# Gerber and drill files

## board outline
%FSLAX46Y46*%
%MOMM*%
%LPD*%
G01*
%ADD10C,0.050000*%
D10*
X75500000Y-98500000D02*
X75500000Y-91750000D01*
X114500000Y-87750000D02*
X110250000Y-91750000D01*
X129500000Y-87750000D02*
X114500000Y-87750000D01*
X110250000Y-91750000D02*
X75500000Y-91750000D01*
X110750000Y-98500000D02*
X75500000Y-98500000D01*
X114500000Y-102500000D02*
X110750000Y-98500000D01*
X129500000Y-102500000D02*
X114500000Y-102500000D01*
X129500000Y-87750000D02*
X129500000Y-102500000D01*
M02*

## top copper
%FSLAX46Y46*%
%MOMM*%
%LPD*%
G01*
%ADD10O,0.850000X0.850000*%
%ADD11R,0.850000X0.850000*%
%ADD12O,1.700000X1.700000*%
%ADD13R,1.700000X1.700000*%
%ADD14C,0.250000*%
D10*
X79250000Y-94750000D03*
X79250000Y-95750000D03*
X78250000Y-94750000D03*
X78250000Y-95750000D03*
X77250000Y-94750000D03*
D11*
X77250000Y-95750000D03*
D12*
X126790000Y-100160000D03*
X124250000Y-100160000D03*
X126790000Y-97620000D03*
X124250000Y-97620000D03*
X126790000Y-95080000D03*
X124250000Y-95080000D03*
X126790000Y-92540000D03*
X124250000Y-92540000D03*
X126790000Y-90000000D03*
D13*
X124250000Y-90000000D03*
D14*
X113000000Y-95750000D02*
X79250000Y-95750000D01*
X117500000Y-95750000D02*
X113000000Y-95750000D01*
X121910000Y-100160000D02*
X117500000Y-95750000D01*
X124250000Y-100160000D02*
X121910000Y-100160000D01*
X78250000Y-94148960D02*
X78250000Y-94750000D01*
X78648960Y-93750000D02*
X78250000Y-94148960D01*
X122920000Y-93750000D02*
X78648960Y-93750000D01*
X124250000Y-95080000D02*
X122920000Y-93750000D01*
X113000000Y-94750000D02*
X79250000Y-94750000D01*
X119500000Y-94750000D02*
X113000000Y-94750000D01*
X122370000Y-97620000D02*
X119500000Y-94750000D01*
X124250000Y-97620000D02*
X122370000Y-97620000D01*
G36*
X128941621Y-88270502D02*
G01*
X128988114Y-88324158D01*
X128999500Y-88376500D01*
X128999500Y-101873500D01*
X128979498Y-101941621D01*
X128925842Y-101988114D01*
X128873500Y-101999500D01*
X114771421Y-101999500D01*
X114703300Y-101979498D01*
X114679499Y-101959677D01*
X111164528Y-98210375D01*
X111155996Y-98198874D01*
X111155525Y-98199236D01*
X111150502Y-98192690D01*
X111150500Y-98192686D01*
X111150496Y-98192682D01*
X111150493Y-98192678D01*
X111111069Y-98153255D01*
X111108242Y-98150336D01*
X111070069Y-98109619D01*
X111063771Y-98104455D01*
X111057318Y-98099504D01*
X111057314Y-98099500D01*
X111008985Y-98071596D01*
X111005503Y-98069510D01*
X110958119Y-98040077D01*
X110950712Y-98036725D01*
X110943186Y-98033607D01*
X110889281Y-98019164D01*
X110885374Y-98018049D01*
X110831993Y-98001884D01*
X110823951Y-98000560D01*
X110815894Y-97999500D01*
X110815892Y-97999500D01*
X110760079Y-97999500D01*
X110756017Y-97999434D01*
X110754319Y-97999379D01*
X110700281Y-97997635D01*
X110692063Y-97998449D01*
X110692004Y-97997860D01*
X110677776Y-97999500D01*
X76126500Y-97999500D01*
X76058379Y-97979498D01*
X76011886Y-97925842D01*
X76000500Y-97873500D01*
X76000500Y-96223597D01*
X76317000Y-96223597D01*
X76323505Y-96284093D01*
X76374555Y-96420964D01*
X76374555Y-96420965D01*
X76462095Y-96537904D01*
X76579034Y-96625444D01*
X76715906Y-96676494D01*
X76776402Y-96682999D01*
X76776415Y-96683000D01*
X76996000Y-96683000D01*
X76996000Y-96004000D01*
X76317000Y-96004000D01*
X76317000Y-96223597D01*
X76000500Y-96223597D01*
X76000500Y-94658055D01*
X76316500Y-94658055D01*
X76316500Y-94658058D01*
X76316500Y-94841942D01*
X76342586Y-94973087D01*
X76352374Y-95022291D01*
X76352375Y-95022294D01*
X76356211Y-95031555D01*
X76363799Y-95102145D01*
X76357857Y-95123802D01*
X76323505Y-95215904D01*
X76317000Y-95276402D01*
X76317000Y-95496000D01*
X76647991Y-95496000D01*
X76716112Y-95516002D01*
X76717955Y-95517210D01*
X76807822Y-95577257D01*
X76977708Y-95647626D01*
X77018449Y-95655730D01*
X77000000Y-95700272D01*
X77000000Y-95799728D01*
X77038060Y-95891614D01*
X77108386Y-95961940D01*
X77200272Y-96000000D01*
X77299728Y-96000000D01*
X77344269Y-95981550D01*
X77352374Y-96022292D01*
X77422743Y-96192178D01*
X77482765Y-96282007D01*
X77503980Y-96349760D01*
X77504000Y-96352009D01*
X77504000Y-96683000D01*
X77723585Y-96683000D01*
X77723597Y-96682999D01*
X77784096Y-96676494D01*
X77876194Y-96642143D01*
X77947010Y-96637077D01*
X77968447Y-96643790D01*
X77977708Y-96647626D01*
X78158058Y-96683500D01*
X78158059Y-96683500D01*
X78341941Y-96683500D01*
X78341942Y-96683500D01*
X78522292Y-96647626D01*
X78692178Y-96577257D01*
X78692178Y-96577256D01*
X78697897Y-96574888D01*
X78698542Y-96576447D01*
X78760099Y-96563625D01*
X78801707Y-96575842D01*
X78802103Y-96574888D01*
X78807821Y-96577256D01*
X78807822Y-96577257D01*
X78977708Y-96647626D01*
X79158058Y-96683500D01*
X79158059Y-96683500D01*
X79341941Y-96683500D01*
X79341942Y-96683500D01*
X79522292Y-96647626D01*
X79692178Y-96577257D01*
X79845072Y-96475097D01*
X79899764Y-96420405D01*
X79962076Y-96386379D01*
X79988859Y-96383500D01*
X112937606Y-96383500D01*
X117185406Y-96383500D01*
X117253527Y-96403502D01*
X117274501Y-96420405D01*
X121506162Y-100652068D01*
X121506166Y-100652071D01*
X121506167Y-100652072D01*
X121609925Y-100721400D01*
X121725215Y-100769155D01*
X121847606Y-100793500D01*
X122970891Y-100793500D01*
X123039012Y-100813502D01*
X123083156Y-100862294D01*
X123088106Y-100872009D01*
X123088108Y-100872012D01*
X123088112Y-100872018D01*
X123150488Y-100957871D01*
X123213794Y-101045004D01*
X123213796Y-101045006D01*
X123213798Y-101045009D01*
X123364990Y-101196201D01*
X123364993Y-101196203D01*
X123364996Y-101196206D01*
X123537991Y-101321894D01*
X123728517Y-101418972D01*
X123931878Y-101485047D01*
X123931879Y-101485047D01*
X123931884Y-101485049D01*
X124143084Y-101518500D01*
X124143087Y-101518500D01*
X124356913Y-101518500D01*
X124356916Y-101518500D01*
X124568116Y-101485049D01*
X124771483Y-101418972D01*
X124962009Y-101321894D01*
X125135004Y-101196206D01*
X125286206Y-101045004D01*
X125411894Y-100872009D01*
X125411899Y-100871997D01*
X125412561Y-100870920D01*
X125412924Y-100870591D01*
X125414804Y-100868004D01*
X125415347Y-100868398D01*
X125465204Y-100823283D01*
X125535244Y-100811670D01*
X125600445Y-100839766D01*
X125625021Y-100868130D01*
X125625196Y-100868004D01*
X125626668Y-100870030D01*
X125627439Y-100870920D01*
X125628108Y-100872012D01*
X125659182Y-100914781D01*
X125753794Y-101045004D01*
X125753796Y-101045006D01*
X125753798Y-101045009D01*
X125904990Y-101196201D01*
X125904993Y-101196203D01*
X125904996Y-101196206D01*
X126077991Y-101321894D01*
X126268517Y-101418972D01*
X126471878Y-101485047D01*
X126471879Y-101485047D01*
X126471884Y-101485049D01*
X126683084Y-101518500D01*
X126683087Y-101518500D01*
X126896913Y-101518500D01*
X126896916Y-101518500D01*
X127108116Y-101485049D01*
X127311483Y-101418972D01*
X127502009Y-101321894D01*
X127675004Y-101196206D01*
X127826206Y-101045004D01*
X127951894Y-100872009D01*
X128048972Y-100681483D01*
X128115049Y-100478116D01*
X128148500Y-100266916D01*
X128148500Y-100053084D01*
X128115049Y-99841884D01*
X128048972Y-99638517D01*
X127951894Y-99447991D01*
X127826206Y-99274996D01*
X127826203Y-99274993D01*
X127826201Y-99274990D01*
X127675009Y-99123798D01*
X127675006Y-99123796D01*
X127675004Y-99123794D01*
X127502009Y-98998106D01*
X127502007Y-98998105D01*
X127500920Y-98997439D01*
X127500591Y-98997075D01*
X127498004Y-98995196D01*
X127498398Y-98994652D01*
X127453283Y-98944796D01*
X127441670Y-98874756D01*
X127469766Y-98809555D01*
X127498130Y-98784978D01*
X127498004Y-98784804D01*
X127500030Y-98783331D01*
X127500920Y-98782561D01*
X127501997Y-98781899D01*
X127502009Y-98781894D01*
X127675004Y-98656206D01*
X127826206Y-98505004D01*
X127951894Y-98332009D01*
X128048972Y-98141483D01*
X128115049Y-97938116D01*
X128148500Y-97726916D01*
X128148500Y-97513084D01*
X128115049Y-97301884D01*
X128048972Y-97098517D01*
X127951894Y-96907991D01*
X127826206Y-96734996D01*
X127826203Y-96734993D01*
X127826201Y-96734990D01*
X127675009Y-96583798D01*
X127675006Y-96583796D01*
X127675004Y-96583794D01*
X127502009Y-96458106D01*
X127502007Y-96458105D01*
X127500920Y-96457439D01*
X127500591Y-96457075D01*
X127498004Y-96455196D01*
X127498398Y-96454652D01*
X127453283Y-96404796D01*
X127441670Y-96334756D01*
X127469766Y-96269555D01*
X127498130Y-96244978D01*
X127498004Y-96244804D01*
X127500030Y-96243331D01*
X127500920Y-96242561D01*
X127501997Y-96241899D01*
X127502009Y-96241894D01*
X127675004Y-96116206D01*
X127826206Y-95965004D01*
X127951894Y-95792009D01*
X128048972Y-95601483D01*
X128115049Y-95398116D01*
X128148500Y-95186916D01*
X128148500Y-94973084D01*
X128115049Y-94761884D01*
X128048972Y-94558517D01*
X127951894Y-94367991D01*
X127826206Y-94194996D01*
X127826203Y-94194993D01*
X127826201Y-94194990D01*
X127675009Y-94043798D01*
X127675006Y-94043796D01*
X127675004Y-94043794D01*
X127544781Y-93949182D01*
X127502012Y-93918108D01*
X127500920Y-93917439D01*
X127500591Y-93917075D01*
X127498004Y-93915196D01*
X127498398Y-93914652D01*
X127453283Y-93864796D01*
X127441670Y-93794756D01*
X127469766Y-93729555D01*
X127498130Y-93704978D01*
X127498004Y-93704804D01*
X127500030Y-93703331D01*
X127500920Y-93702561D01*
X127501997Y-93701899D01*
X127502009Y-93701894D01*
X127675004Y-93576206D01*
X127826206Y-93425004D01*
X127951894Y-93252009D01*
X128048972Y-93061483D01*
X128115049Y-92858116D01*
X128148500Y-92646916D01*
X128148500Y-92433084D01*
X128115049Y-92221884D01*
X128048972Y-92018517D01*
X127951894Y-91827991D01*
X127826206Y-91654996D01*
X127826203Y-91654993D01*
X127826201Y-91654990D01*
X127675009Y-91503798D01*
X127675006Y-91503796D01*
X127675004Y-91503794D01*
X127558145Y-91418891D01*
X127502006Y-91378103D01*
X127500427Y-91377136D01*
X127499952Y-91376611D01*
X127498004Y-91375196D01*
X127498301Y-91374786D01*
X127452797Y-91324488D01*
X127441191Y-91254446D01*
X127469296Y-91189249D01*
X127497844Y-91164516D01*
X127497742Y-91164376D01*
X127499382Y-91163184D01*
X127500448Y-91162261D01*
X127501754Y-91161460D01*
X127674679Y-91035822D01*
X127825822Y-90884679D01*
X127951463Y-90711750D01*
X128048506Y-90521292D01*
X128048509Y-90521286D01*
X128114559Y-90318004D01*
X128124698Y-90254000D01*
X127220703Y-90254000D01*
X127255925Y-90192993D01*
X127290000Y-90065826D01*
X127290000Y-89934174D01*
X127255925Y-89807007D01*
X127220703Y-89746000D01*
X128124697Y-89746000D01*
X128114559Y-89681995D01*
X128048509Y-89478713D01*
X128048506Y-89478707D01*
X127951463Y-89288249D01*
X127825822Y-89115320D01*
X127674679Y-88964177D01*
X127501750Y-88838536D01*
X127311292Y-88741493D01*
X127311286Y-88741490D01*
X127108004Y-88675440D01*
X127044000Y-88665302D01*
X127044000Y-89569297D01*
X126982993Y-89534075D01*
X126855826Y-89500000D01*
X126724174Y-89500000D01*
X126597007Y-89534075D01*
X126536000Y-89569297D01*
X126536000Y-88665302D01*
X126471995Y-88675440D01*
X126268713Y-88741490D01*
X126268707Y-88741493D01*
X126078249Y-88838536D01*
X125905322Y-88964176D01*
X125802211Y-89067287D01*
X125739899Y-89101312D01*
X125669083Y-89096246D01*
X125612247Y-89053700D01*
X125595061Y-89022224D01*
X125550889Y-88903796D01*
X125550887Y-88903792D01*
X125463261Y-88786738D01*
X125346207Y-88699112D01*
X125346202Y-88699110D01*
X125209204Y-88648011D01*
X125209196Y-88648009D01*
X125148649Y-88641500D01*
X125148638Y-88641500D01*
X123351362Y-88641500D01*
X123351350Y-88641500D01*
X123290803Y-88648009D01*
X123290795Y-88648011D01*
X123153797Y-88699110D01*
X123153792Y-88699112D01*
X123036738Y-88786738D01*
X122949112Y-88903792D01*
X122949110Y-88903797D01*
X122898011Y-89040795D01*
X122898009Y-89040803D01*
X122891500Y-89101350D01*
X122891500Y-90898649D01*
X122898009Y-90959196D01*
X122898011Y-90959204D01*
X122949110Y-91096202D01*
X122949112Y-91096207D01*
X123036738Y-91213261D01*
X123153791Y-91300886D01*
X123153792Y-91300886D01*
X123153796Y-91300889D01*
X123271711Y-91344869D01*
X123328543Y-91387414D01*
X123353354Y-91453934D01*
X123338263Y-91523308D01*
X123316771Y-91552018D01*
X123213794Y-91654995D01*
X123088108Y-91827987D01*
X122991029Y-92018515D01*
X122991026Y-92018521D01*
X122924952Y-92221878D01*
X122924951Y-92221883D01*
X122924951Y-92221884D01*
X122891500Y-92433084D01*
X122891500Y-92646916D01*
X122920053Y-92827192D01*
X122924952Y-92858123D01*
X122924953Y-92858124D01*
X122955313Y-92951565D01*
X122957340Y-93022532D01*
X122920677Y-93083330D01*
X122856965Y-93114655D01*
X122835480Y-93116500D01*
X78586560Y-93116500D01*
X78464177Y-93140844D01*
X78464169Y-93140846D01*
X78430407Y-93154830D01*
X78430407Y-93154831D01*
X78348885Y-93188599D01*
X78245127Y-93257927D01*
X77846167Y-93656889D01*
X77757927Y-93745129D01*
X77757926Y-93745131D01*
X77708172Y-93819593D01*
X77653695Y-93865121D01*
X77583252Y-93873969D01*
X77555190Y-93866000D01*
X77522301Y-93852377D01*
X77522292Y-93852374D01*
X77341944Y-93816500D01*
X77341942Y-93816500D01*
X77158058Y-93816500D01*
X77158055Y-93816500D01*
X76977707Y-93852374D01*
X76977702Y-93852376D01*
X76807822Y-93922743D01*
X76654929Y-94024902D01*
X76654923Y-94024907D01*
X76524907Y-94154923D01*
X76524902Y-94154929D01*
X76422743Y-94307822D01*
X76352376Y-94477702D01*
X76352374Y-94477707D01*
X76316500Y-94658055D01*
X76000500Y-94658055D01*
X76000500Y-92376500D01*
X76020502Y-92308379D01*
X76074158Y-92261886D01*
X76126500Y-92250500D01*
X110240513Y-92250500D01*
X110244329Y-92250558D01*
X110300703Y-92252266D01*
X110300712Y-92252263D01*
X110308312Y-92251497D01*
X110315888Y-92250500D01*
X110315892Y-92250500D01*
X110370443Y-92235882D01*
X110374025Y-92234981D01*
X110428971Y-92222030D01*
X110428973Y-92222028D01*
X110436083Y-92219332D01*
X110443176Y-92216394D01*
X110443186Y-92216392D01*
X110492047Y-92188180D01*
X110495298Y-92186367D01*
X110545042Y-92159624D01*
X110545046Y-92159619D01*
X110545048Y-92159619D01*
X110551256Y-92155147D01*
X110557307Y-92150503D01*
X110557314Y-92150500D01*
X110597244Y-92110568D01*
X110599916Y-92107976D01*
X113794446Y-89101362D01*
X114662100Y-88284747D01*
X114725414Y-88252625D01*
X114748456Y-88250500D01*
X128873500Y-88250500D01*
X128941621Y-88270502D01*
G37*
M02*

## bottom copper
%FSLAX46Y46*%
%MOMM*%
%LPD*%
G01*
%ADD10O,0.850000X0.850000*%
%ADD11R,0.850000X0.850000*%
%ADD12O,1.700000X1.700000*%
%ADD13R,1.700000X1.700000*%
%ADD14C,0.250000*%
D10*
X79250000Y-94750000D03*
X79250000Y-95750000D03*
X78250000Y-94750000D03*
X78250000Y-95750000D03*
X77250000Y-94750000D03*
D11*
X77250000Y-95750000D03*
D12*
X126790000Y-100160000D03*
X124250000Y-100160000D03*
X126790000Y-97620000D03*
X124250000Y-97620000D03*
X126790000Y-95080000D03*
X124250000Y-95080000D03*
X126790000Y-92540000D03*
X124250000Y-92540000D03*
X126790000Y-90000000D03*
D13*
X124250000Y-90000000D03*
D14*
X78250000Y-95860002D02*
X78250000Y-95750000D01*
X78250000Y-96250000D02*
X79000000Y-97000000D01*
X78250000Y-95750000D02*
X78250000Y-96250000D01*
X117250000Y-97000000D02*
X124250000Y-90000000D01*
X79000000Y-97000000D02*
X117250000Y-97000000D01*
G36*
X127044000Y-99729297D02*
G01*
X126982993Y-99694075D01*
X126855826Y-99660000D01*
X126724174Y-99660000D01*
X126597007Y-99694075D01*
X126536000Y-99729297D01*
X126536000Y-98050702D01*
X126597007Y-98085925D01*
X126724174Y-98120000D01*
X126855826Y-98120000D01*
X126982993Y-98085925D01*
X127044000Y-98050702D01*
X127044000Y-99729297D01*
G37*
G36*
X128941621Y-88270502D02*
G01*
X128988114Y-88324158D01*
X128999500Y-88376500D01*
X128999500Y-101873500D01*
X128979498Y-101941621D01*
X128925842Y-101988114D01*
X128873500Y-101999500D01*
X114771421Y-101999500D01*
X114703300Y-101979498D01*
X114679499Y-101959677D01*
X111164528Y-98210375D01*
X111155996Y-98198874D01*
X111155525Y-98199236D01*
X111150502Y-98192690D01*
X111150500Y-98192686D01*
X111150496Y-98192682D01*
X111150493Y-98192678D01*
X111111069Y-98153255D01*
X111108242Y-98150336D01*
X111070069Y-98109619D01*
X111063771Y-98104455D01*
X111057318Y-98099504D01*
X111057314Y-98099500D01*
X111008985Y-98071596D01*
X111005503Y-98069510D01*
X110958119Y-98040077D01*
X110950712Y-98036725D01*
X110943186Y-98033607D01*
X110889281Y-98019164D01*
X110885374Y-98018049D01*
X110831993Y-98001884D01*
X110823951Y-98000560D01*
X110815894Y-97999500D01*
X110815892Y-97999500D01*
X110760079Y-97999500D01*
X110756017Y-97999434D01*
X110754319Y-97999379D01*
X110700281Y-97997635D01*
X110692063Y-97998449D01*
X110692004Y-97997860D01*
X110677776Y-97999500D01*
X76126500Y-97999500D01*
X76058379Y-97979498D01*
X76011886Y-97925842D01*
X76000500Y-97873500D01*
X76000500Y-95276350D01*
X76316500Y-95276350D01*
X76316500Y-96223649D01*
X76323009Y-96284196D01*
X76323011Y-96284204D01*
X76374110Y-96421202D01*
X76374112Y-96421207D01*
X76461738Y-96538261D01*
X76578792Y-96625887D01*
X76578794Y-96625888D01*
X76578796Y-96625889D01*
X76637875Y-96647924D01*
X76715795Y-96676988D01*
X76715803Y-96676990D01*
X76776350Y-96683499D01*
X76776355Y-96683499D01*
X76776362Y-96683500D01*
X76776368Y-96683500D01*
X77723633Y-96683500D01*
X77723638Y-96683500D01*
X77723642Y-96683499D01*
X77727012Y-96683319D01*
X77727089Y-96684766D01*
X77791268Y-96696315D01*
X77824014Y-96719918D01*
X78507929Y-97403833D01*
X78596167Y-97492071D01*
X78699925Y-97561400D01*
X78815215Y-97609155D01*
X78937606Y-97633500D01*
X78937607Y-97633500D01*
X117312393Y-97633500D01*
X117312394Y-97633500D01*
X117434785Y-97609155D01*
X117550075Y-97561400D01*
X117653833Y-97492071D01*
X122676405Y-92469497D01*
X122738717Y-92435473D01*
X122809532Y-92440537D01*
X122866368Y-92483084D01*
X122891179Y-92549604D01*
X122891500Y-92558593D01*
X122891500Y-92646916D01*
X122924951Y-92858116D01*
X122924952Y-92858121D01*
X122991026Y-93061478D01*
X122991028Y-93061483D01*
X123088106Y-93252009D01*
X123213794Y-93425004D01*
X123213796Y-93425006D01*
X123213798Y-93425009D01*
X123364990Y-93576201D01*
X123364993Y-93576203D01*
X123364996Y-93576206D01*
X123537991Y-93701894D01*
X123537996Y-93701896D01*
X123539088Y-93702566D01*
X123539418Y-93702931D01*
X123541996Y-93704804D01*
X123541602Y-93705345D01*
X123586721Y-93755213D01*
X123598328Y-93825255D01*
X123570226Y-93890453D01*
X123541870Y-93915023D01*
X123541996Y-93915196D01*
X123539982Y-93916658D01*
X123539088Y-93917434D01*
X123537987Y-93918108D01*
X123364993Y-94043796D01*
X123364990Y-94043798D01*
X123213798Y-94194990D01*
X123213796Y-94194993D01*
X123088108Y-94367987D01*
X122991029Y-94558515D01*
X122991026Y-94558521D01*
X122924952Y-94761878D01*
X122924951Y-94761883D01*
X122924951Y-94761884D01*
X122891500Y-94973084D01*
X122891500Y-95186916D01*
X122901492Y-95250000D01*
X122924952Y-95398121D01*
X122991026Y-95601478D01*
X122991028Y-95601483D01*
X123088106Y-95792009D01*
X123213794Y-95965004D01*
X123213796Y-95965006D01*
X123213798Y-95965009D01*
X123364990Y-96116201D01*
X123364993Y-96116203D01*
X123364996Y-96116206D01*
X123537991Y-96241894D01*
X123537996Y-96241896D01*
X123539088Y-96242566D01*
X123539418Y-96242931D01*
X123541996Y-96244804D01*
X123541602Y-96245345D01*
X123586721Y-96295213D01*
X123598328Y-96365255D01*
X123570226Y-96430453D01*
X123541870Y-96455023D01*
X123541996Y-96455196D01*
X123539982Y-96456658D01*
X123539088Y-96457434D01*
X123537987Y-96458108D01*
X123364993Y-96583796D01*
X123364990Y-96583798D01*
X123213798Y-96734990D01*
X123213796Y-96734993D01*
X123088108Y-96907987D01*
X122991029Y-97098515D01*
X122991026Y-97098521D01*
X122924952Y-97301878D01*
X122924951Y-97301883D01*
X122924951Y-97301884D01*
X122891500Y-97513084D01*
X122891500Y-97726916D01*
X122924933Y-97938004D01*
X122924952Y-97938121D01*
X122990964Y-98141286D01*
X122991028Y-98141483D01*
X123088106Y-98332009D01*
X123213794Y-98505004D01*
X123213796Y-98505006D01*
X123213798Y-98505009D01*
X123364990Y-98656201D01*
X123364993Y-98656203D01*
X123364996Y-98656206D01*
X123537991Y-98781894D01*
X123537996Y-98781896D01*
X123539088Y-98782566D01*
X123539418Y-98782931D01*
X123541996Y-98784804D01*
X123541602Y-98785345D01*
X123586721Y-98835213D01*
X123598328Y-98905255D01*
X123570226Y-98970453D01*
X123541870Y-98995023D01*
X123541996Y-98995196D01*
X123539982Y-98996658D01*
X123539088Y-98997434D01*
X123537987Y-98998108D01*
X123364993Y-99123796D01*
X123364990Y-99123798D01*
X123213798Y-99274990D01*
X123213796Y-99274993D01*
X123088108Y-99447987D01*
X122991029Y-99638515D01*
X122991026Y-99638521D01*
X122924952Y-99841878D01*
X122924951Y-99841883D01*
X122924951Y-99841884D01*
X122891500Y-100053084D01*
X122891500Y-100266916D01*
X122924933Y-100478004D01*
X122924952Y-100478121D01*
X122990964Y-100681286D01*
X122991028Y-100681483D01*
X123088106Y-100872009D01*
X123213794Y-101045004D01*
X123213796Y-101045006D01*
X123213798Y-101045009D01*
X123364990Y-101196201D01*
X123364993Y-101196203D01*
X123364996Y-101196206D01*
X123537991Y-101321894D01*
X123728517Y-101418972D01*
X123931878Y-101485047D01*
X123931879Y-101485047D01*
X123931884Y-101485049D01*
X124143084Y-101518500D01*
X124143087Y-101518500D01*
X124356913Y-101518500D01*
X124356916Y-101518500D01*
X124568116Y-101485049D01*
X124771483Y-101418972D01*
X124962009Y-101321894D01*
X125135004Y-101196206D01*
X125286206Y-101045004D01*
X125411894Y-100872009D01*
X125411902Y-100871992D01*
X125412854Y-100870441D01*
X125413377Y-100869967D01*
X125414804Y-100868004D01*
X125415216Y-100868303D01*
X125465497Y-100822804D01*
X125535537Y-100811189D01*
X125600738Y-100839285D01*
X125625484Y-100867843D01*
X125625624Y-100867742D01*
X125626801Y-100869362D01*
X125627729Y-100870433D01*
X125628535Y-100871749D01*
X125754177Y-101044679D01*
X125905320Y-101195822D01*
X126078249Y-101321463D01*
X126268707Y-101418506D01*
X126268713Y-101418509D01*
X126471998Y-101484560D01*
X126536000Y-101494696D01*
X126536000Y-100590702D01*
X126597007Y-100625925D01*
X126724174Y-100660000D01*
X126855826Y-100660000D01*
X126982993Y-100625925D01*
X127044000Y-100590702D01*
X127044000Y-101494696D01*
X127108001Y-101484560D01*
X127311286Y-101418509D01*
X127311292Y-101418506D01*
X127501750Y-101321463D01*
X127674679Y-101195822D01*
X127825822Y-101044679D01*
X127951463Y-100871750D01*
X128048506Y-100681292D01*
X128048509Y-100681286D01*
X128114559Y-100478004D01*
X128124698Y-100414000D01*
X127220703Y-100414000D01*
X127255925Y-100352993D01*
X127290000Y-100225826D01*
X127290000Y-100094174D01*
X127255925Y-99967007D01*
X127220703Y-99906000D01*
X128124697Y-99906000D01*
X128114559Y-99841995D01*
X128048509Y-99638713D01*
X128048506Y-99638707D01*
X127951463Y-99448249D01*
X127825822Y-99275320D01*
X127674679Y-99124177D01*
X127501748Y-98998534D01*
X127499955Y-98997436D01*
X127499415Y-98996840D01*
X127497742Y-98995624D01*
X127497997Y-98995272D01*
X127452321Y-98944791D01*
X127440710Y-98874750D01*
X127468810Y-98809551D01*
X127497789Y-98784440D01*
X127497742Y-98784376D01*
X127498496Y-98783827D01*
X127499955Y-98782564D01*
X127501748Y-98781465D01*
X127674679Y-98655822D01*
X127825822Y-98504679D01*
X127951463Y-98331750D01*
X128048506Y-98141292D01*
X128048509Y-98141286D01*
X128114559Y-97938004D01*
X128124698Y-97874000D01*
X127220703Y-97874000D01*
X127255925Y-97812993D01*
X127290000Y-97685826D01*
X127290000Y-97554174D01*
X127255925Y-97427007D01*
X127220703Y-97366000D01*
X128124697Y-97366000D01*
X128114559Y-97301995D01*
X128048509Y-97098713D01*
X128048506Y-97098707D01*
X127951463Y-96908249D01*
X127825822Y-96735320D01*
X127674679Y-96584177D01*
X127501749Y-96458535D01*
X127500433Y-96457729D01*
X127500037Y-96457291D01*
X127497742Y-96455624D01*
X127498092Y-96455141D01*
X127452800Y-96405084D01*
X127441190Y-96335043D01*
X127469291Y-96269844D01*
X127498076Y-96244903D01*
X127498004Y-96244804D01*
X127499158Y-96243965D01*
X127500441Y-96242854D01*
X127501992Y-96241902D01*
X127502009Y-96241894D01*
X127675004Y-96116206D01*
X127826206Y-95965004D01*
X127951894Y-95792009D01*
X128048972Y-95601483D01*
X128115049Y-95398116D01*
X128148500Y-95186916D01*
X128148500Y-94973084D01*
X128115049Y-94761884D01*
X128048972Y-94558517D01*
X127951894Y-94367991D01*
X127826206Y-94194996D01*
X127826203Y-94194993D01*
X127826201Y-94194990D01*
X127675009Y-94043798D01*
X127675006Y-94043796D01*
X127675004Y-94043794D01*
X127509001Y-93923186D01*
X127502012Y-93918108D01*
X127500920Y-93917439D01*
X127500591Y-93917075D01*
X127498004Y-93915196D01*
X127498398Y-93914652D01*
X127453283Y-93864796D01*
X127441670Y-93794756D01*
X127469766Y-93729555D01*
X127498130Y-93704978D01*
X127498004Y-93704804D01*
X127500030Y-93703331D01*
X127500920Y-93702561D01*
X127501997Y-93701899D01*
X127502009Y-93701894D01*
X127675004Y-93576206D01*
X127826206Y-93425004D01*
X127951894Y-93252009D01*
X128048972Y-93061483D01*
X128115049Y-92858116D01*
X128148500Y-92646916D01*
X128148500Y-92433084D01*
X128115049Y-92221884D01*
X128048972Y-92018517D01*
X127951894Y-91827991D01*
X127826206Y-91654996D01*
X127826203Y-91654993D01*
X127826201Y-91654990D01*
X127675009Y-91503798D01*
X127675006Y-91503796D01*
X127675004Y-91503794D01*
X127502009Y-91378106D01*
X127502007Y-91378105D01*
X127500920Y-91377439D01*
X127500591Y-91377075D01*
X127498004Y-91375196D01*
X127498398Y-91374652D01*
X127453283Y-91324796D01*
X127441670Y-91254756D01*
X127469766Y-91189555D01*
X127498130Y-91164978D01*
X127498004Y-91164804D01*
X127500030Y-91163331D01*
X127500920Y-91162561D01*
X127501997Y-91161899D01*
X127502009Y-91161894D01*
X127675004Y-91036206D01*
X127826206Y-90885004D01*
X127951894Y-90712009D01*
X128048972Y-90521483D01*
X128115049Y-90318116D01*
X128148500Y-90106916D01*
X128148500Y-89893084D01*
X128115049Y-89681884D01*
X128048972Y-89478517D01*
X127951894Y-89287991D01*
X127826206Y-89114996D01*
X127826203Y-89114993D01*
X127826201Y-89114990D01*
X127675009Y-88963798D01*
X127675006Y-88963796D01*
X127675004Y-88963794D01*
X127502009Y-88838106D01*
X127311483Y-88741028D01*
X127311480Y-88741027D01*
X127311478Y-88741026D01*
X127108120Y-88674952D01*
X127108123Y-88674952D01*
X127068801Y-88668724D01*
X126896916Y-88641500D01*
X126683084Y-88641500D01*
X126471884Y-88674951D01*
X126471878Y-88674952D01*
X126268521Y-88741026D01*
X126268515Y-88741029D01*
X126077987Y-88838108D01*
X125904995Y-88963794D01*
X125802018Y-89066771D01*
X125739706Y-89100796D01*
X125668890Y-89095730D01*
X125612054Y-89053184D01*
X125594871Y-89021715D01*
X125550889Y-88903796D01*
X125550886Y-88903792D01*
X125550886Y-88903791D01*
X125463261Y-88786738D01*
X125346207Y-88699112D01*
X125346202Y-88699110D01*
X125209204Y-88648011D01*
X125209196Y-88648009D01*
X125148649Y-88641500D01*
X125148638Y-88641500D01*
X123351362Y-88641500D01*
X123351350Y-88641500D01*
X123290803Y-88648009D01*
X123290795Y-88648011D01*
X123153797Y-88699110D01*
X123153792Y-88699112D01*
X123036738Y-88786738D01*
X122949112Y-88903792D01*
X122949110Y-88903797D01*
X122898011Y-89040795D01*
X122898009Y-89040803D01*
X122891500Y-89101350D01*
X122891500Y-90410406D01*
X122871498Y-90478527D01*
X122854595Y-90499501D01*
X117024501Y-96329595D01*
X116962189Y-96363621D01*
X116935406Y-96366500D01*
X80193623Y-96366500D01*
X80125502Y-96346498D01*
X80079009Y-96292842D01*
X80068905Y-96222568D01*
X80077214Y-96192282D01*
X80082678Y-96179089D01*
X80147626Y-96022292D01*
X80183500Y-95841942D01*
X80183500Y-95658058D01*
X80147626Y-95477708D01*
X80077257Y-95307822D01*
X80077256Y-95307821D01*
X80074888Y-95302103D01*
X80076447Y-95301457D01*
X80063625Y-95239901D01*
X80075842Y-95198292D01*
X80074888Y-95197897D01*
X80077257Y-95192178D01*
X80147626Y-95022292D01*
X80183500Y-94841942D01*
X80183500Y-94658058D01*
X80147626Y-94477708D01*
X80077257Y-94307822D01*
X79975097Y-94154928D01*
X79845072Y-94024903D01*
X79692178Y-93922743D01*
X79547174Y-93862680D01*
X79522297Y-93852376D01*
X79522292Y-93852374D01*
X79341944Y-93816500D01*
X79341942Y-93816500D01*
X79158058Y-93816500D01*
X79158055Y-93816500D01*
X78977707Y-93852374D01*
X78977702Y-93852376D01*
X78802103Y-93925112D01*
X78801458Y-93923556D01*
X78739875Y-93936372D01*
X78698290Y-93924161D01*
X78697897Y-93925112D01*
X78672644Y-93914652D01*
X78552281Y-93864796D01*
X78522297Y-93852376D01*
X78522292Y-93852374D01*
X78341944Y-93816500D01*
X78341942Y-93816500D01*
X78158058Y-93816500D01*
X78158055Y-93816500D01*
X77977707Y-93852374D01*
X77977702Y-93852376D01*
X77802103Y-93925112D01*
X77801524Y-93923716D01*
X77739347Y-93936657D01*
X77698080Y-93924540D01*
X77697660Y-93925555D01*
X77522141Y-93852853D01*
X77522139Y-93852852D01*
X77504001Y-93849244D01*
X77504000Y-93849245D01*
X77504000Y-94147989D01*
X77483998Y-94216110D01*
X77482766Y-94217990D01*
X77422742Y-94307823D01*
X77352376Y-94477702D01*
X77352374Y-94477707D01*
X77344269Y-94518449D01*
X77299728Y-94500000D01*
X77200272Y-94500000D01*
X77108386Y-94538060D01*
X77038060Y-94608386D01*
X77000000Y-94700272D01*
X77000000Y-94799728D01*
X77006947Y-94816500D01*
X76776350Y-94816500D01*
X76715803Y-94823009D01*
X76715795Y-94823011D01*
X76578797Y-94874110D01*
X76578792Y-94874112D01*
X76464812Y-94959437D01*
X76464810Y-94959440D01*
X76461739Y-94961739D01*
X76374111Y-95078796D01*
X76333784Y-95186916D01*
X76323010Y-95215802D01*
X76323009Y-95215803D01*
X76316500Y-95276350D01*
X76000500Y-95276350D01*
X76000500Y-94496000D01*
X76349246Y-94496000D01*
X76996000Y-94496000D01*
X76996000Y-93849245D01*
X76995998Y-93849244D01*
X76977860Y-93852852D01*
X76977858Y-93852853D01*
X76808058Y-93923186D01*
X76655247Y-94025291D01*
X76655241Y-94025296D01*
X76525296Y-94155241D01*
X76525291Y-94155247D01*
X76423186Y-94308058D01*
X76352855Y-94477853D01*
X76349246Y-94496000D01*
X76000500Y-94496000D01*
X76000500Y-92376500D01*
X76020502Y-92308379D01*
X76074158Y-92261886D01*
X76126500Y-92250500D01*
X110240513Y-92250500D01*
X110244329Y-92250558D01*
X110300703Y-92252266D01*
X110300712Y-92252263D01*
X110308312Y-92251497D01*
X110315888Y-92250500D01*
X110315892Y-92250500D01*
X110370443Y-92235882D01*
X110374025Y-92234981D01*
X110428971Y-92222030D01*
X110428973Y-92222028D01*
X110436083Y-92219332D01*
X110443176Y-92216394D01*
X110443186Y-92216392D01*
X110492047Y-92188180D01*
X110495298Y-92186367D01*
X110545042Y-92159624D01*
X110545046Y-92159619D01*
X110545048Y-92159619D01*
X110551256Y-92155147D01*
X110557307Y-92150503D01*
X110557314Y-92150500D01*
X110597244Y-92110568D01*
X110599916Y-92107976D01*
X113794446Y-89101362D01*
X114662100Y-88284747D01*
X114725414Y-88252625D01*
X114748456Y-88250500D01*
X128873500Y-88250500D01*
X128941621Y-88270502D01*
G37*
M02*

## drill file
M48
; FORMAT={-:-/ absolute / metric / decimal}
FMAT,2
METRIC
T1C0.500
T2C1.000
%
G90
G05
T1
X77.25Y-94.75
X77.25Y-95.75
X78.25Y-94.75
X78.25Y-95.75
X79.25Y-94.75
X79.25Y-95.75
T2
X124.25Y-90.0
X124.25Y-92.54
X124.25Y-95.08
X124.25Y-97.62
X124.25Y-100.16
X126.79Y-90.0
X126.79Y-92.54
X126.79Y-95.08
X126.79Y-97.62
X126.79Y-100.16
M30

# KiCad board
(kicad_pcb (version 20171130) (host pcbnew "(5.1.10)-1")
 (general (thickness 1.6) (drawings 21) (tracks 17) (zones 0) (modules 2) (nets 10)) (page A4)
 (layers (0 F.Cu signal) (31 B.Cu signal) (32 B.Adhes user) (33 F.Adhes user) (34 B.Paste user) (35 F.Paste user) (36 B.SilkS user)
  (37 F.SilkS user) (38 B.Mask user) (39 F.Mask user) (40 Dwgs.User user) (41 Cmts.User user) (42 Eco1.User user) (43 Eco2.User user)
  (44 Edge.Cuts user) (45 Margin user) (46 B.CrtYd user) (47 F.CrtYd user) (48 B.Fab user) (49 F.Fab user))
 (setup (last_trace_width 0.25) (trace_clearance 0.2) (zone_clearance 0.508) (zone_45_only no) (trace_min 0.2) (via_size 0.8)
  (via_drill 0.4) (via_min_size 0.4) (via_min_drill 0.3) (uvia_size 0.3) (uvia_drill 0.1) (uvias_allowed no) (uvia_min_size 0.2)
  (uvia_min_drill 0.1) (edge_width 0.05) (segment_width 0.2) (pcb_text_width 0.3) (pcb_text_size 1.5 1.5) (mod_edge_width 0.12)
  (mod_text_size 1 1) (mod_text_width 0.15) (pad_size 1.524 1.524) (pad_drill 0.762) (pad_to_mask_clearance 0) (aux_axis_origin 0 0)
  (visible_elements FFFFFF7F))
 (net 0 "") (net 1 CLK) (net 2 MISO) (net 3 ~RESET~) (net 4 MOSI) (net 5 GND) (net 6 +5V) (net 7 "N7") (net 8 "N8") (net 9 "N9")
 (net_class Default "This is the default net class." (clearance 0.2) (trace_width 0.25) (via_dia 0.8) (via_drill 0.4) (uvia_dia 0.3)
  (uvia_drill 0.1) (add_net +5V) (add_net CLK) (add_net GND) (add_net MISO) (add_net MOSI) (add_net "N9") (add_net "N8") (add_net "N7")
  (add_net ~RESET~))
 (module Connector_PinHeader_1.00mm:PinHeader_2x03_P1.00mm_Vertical (layer F.Cu) (at 77.25 95.75 90)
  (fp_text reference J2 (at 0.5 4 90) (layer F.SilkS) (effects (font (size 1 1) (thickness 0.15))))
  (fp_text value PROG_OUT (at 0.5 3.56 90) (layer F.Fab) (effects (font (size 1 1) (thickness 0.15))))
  (pad 6 thru_hole oval (at 1 2 90) (size 0.85 0.85) (drill 0.5) (layers *.Cu *.Mask) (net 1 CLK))
  (pad 5 thru_hole oval (at 0 2 90) (size 0.85 0.85) (drill 0.5) (layers *.Cu *.Mask) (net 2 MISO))
  (pad 4 thru_hole oval (at 1 1 90) (size 0.85 0.85) (drill 0.5) (layers *.Cu *.Mask) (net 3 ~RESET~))
  (pad 3 thru_hole oval (at 0 1 90) (size 0.85 0.85) (drill 0.5) (layers *.Cu *.Mask) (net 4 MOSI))
  (pad 2 thru_hole oval (at 1 0 90) (size 0.85 0.85) (drill 0.5) (layers *.Cu *.Mask) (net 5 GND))
  (pad 1 thru_hole rect (at 0 0 90) (size 0.85 0.85) (drill 0.5) (layers *.Cu *.Mask) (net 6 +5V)))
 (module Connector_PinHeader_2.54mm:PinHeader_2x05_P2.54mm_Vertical (layer F.Cu) (at 124.25 90)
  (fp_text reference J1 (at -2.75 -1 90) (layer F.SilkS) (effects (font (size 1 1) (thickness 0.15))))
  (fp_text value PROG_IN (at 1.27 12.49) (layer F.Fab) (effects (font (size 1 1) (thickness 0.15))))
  (pad 10 thru_hole oval (at 2.54 10.16) (size 1.7 1.7) (drill 1) (layers *.Cu *.Mask) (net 5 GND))
  (pad 9 thru_hole oval (at 0 10.16) (size 1.7 1.7) (drill 1) (layers *.Cu *.Mask) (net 2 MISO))
  (pad 8 thru_hole oval (at 2.54 7.62) (size 1.7 1.7) (drill 1) (layers *.Cu *.Mask) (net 5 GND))
  (pad 7 thru_hole oval (at 0 7.62) (size 1.7 1.7) (drill 1) (layers *.Cu *.Mask) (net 1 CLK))
  (pad 6 thru_hole oval (at 2.54 5.08) (size 1.7 1.7) (drill 1) (layers *.Cu *.Mask) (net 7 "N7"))
  (pad 5 thru_hole oval (at 0 5.08) (size 1.7 1.7) (drill 1) (layers *.Cu *.Mask) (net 3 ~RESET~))
  (pad 4 thru_hole oval (at 2.54 2.54) (size 1.7 1.7) (drill 1) (layers *.Cu *.Mask) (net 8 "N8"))
  (pad 3 thru_hole oval (at 0 2.54) (size 1.7 1.7) (drill 1) (layers *.Cu *.Mask) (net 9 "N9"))
  (pad 2 thru_hole oval (at 2.54 0) (size 1.7 1.7) (drill 1) (layers *.Cu *.Mask) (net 6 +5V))
  (pad 1 thru_hole rect (at 0 0) (size 1.7 1.7) (drill 1) (layers *.Cu *.Mask) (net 4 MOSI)))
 (gr_line (start 75.5 98.5) (end 75.5 91.75) (layer Edge.Cuts) (width 0.05))
 (gr_line (start 114.5 87.75) (end 110.25 91.75) (layer Edge.Cuts) (width 0.05))
 (gr_line (start 129.5 87.75) (end 114.5 87.75) (layer Edge.Cuts) (width 0.05))
 (gr_line (start 110.25 91.75) (end 75.5 91.75) (layer Edge.Cuts) (width 0.05))
 (gr_line (start 110.75 98.5) (end 75.5 98.5) (layer Edge.Cuts) (width 0.05))
 (gr_line (start 114.5 102.5) (end 110.75 98.5) (layer Edge.Cuts) (width 0.05))
 (gr_line (start 129.5 102.5) (end 114.5 102.5) (layer Edge.Cuts) (width 0.05))
 (gr_line (start 129.5 87.75) (end 129.5 102.5) (layer Edge.Cuts) (width 0.05))
 (segment (start 113 95.75) (end 79.25 95.75) (width 0.25) (layer F.Cu) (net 2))
 (segment (start 117.5 95.75) (end 113 95.75) (width 0.25) (layer F.Cu) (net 2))
 (segment (start 121.91 100.16) (end 117.5 95.75) (width 0.25) (layer F.Cu) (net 2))
 (segment (start 124.25 100.16) (end 121.91 100.16) (width 0.25) (layer F.Cu) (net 2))
 (segment (start 78.25 94.14896) (end 78.25 94.75) (width 0.25) (layer F.Cu) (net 3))
 (segment (start 78.64896 93.75) (end 78.25 94.14896) (width 0.25) (layer F.Cu) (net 3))
 (segment (start 122.92 93.75) (end 78.64896 93.75) (width 0.25) (layer F.Cu) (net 3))
 (segment (start 124.25 95.08) (end 122.92 93.75) (width 0.25) (layer F.Cu) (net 3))
 (segment (start 78.25 95.860002) (end 78.25 95.75) (width 0.25) (layer B.Cu) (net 4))
 (segment (start 78.25 96.25) (end 79 97) (width 0.25) (layer B.Cu) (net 4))
 (segment (start 78.25 95.75) (end 78.25 96.25) (width 0.25) (layer B.Cu) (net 4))
 (segment (start 117.25 97) (end 124.25 90) (width 0.25) (layer B.Cu) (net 4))
 (segment (start 79 97) (end 117.25 97) (width 0.25) (layer B.Cu) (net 4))
 (segment (start 113 94.75) (end 79.25 94.75) (width 0.25) (layer F.Cu) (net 1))
 (segment (start 119.5 94.75) (end 113 94.75) (width 0.25) (layer F.Cu) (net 1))
 (segment (start 122.37 97.62) (end 119.5 94.75) (width 0.25) (layer F.Cu) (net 1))
 (segment (start 124.25 97.62) (end 122.37 97.62) (width 0.25) (layer F.Cu) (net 1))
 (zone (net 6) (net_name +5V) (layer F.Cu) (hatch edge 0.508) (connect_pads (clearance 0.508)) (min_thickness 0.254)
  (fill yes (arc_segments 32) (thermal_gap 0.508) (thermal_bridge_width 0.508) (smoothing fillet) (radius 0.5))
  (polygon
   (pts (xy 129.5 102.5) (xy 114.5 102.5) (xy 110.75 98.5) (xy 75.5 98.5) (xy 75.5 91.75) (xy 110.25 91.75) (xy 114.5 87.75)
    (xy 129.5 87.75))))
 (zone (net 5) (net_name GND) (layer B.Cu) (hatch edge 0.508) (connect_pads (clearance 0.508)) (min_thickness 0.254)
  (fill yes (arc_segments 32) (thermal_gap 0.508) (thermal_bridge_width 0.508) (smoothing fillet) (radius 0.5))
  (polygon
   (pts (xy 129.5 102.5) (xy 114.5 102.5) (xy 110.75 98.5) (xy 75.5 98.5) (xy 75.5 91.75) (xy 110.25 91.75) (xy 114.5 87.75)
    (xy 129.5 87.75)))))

